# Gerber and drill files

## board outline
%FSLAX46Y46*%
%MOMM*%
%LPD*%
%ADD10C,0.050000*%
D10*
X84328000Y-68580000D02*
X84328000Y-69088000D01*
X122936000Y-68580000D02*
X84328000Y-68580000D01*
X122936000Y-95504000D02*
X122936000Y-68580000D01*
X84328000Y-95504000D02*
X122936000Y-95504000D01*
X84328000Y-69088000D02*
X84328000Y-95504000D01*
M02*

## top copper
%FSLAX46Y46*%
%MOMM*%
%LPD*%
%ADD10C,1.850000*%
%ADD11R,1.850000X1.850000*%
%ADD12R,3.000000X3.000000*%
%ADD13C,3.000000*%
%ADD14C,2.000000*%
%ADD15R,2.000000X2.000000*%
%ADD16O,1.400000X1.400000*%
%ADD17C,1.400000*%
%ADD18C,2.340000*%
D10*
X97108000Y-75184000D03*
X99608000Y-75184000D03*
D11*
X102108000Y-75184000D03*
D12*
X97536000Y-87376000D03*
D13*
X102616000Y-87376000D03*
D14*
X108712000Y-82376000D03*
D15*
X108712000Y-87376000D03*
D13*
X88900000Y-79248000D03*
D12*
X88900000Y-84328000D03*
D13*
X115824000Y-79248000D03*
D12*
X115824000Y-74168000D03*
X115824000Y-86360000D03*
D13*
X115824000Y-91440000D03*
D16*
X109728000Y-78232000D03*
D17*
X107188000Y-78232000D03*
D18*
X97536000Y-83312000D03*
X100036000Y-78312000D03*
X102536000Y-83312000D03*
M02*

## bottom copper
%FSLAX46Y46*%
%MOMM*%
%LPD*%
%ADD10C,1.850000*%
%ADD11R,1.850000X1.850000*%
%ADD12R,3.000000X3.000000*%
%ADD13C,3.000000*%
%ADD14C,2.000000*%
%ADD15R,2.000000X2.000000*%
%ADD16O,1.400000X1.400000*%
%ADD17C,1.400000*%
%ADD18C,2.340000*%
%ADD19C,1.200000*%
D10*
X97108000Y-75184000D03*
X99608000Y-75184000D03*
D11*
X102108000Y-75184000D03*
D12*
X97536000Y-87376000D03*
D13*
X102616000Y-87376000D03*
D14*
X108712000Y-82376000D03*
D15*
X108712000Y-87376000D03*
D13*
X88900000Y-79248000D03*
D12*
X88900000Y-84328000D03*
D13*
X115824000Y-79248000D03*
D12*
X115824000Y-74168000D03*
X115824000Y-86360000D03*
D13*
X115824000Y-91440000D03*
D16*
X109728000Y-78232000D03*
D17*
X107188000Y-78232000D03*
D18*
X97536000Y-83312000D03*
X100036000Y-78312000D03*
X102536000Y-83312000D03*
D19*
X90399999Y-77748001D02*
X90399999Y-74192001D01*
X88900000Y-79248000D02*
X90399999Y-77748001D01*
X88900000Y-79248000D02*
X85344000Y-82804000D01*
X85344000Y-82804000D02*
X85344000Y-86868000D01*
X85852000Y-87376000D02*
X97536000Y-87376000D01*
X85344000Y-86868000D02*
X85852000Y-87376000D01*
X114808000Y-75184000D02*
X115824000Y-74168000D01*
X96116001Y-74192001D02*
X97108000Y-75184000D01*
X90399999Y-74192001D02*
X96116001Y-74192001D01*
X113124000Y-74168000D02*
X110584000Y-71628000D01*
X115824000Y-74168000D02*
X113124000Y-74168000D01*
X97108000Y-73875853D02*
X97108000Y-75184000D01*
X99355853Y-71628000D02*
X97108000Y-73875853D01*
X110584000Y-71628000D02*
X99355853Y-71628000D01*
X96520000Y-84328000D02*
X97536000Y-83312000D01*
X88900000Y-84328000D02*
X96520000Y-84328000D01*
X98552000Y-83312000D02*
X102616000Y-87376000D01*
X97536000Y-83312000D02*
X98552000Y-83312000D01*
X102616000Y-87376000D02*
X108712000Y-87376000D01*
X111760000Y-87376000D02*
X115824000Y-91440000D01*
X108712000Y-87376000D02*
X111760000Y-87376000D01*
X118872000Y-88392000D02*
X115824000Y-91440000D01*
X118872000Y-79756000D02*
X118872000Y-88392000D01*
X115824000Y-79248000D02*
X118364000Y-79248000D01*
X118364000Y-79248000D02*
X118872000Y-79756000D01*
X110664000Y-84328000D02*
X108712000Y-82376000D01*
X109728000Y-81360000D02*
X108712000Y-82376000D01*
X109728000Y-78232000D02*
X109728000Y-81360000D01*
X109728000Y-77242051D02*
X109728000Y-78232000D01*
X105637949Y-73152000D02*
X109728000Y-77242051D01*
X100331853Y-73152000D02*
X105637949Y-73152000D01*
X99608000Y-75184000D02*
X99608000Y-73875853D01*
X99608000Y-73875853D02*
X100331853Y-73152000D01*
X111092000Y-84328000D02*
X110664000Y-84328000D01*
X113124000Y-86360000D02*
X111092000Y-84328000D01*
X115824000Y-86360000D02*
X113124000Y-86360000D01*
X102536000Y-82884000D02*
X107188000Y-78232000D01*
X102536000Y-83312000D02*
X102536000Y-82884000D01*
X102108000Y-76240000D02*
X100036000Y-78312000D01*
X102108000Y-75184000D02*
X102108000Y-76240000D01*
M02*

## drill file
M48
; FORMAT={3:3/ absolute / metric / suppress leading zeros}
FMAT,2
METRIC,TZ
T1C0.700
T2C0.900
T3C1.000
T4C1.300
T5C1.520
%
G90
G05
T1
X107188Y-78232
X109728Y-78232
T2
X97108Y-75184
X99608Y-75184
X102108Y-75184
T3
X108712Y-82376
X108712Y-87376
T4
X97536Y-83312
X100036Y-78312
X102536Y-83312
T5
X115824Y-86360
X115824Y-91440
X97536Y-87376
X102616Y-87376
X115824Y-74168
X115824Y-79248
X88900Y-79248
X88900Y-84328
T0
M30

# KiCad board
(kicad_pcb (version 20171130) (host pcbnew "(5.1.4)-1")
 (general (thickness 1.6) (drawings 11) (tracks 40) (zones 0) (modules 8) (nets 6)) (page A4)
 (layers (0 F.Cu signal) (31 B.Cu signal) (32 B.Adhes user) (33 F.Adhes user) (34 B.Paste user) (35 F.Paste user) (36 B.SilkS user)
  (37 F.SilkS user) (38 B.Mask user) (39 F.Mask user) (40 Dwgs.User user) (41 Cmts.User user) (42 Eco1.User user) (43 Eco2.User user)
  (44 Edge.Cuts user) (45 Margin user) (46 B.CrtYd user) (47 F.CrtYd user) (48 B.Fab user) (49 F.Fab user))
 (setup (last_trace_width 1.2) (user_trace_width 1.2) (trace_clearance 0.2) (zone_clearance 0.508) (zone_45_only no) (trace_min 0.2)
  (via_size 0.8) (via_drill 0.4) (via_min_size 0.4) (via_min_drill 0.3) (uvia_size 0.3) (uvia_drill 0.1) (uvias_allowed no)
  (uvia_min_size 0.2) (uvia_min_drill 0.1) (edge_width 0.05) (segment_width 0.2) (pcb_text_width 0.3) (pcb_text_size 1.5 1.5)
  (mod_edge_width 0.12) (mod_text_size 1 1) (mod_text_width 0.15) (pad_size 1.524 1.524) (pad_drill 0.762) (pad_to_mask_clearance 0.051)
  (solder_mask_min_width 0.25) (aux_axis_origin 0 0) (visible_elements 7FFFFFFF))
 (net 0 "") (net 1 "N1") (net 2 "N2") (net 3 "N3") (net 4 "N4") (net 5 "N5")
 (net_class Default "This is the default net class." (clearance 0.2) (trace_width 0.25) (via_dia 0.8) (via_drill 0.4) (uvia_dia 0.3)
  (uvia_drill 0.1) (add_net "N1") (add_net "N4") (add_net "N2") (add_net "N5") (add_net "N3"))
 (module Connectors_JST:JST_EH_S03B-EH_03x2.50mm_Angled (layer F.Cu) (at 102.108 75.184 180)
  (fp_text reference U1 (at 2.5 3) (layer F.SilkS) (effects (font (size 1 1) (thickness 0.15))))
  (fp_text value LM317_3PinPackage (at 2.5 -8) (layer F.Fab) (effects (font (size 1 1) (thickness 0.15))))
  (pad 3 thru_hole circle (at 5 0 180) (size 1.85 1.85) (drill 0.9) (layers *.Cu *.Mask) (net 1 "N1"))
  (pad 2 thru_hole circle (at 2.5 0 180) (size 1.85 1.85) (drill 0.9) (layers *.Cu *.Mask) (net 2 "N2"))
  (pad 1 thru_hole rect (at 0 0 180) (size 1.85 1.85) (drill 0.9) (layers *.Cu *.Mask) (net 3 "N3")))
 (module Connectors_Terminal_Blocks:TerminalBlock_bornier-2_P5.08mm (layer F.Cu) (at 97.536 87.376)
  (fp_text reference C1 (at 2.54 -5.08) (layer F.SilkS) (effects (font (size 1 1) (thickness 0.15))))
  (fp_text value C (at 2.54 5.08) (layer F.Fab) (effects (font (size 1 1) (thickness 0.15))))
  (pad 1 thru_hole rect (at 0 0) (size 3 3) (drill 1.52) (layers *.Cu *.Mask) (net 1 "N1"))
  (pad 2 thru_hole circle (at 5.08 0) (size 3 3) (drill 1.52) (layers *.Cu *.Mask) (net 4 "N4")))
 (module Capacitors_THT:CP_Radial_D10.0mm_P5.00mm (layer F.Cu) (at 108.712 87.376 90)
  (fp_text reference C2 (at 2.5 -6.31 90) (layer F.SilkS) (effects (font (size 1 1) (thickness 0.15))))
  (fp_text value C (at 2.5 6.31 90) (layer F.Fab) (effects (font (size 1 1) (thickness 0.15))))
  (pad 2 thru_hole circle (at 5 0 90) (size 2 2) (drill 1) (layers *.Cu *.Mask) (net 2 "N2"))
  (pad 1 thru_hole rect (at 0 0 90) (size 2 2) (drill 1) (layers *.Cu *.Mask) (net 4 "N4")))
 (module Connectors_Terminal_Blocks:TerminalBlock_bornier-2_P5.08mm (layer F.Cu) (at 88.9 84.328 90)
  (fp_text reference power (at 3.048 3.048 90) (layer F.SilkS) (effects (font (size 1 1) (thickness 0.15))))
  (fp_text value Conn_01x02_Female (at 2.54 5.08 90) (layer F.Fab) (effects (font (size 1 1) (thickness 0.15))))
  (pad 2 thru_hole circle (at 5.08 0 90) (size 3 3) (drill 1.52) (layers *.Cu *.Mask) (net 1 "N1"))
  (pad 1 thru_hole rect (at 0 0 90) (size 3 3) (drill 1.52) (layers *.Cu *.Mask) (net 4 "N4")))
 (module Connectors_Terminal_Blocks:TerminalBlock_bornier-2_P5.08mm (layer F.Cu) (at 115.824 74.168 270)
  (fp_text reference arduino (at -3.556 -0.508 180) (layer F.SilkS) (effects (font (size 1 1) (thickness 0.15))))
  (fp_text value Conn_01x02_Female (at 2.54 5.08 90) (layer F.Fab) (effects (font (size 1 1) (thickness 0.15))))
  (pad 2 thru_hole circle (at 5.08 0 270) (size 3 3) (drill 1.52) (layers *.Cu *.Mask) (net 4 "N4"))
  (pad 1 thru_hole rect (at 0 0 270) (size 3 3) (drill 1.52) (layers *.Cu *.Mask) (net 1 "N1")))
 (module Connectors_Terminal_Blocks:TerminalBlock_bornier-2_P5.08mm (layer F.Cu) (at 115.824 86.36 270)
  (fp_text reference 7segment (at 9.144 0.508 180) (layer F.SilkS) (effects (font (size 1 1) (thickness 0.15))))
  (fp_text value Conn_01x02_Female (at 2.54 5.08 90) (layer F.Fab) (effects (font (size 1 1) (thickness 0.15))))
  (pad 1 thru_hole rect (at 0 0 270) (size 3 3) (drill 1.52) (layers *.Cu *.Mask) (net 2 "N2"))
  (pad 2 thru_hole circle (at 5.08 0 270) (size 3 3) (drill 1.52) (layers *.Cu *.Mask) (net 4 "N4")))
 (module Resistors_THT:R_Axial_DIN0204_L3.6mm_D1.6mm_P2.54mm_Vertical (layer F.Cu) (at 107.188 78.232)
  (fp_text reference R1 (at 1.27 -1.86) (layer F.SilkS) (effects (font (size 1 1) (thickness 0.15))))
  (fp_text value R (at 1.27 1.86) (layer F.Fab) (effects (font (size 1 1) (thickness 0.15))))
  (pad 2 thru_hole oval (at 2.54 0) (size 1.4 1.4) (drill 0.7) (layers *.Cu *.Mask) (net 2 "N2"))
  (pad 1 thru_hole circle (at 0 0) (size 1.4 1.4) (drill 0.7) (layers *.Cu *.Mask) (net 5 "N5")))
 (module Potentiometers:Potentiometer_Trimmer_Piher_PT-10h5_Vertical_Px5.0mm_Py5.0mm (layer F.Cu) (at 97.536 83.312 90)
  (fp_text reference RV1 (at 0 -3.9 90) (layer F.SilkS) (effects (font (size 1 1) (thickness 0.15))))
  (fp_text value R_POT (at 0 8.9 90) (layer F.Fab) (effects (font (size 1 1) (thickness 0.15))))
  (pad 1 thru_hole circle (at 0 0 90) (size 2.34 2.34) (drill 1.3) (layers *.Cu *.Mask) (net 4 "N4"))
  (pad 2 thru_hole circle (at 5 2.5 90) (size 2.34 2.34) (drill 1.3) (layers *.Cu *.Mask) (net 3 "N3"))
  (pad 3 thru_hole circle (at 0 5 90) (size 2.34 2.34) (drill 1.3) (layers *.Cu *.Mask) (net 5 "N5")))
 (gr_line (start 84.328 68.58) (end 84.328 69.088) (layer Edge.Cuts) (width 0.05))
 (gr_line (start 122.936 68.58) (end 84.328 68.58) (layer Edge.Cuts) (width 0.05))
 (gr_line (start 122.936 95.504) (end 122.936 68.58) (layer Edge.Cuts) (width 0.05))
 (gr_line (start 84.328 95.504) (end 122.936 95.504) (layer Edge.Cuts) (width 0.05))
 (gr_line (start 84.328 69.088) (end 84.328 95.504) (layer Edge.Cuts) (width 0.05))
 (segment (start 90.399999 77.748001) (end 90.399999 74.192001) (width 1.2) (layer B.Cu) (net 1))
 (segment (start 88.9 79.248) (end 90.399999 77.748001) (width 1.2) (layer B.Cu) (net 1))
 (segment (start 88.9 79.248) (end 85.344 82.804) (width 1.2) (layer B.Cu) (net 1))
 (segment (start 85.344 82.804) (end 85.344 86.868) (width 1.2) (layer B.Cu) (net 1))
 (segment (start 85.852 87.376) (end 97.536 87.376) (width 1.2) (layer B.Cu) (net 1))
 (segment (start 85.344 86.868) (end 85.852 87.376) (width 1.2) (layer B.Cu) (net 1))
 (segment (start 114.808 75.184) (end 115.824 74.168) (width 1.2) (layer B.Cu) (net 1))
 (segment (start 96.116001 74.192001) (end 97.108 75.184) (width 1.2) (layer B.Cu) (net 1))
 (segment (start 90.399999 74.192001) (end 96.116001 74.192001) (width 1.2) (layer B.Cu) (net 1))
 (segment (start 113.124 74.168) (end 110.584 71.628) (width 1.2) (layer B.Cu) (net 1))
 (segment (start 115.824 74.168) (end 113.124 74.168) (width 1.2) (layer B.Cu) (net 1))
 (segment (start 97.108 73.875853) (end 97.108 75.184) (width 1.2) (layer B.Cu) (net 1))
 (segment (start 99.355853 71.628) (end 97.108 73.875853) (width 1.2) (layer B.Cu) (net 1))
 (segment (start 110.584 71.628) (end 99.355853 71.628) (width 1.2) (layer B.Cu) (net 1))
 (segment (start 96.52 84.328) (end 97.536 83.312) (width 1.2) (layer B.Cu) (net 4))
 (segment (start 88.9 84.328) (end 96.52 84.328) (width 1.2) (layer B.Cu) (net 4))
 (segment (start 98.552 83.312) (end 102.616 87.376) (width 1.2) (layer B.Cu) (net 4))
 (segment (start 97.536 83.312) (end 98.552 83.312) (width 1.2) (layer B.Cu) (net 4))
 (segment (start 102.616 87.376) (end 108.712 87.376) (width 1.2) (layer B.Cu) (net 4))
 (segment (start 111.76 87.376) (end 115.824 91.44) (width 1.2) (layer B.Cu) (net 4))
 (segment (start 108.712 87.376) (end 111.76 87.376) (width 1.2) (layer B.Cu) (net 4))
 (segment (start 118.872 88.392) (end 115.824 91.44) (width 1.2) (layer B.Cu) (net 4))
 (segment (start 118.872 79.756) (end 118.872 88.392) (width 1.2) (layer B.Cu) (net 4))
 (segment (start 115.824 79.248) (end 118.364 79.248) (width 1.2) (layer B.Cu) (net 4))
 (segment (start 118.364 79.248) (end 118.872 79.756) (width 1.2) (layer B.Cu) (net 4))
 (segment (start 110.664 84.328) (end 108.712 82.376) (width 1.2) (layer B.Cu) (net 2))
 (segment (start 109.728 81.36) (end 108.712 82.376) (width 1.2) (layer B.Cu) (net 2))
 (segment (start 109.728 78.232) (end 109.728 81.36) (width 1.2) (layer B.Cu) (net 2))
 (segment (start 109.728 77.242051) (end 109.728 78.232) (width 1.2) (layer B.Cu) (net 2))
 (segment (start 105.637949 73.152) (end 109.728 77.242051) (width 1.2) (layer B.Cu) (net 2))
 (segment (start 100.331853 73.152) (end 105.637949 73.152) (width 1.2) (layer B.Cu) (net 2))
 (segment (start 99.608 75.184) (end 99.608 73.875853) (width 1.2) (layer B.Cu) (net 2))
 (segment (start 99.608 73.875853) (end 100.331853 73.152) (width 1.2) (layer B.Cu) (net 2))
 (segment (start 111.092 84.328) (end 110.664 84.328) (width 1.2) (layer B.Cu) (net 2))
 (segment (start 113.124 86.36) (end 111.092 84.328) (width 1.2) (layer B.Cu) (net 2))
 (segment (start 115.824 86.36) (end 113.124 86.36) (width 1.2) (layer B.Cu) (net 2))
 (segment (start 102.536 82.884) (end 107.188 78.232) (width 1.2) (layer B.Cu) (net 5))
 (segment (start 102.536 83.312) (end 102.536 82.884) (width 1.2) (layer B.Cu) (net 5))
 (segment (start 102.108 76.24) (end 100.036 78.312) (width 1.2) (layer B.Cu) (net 3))
 (segment (start 102.108 75.184) (end 102.108 76.24) (width 1.2) (layer B.Cu) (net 3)))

